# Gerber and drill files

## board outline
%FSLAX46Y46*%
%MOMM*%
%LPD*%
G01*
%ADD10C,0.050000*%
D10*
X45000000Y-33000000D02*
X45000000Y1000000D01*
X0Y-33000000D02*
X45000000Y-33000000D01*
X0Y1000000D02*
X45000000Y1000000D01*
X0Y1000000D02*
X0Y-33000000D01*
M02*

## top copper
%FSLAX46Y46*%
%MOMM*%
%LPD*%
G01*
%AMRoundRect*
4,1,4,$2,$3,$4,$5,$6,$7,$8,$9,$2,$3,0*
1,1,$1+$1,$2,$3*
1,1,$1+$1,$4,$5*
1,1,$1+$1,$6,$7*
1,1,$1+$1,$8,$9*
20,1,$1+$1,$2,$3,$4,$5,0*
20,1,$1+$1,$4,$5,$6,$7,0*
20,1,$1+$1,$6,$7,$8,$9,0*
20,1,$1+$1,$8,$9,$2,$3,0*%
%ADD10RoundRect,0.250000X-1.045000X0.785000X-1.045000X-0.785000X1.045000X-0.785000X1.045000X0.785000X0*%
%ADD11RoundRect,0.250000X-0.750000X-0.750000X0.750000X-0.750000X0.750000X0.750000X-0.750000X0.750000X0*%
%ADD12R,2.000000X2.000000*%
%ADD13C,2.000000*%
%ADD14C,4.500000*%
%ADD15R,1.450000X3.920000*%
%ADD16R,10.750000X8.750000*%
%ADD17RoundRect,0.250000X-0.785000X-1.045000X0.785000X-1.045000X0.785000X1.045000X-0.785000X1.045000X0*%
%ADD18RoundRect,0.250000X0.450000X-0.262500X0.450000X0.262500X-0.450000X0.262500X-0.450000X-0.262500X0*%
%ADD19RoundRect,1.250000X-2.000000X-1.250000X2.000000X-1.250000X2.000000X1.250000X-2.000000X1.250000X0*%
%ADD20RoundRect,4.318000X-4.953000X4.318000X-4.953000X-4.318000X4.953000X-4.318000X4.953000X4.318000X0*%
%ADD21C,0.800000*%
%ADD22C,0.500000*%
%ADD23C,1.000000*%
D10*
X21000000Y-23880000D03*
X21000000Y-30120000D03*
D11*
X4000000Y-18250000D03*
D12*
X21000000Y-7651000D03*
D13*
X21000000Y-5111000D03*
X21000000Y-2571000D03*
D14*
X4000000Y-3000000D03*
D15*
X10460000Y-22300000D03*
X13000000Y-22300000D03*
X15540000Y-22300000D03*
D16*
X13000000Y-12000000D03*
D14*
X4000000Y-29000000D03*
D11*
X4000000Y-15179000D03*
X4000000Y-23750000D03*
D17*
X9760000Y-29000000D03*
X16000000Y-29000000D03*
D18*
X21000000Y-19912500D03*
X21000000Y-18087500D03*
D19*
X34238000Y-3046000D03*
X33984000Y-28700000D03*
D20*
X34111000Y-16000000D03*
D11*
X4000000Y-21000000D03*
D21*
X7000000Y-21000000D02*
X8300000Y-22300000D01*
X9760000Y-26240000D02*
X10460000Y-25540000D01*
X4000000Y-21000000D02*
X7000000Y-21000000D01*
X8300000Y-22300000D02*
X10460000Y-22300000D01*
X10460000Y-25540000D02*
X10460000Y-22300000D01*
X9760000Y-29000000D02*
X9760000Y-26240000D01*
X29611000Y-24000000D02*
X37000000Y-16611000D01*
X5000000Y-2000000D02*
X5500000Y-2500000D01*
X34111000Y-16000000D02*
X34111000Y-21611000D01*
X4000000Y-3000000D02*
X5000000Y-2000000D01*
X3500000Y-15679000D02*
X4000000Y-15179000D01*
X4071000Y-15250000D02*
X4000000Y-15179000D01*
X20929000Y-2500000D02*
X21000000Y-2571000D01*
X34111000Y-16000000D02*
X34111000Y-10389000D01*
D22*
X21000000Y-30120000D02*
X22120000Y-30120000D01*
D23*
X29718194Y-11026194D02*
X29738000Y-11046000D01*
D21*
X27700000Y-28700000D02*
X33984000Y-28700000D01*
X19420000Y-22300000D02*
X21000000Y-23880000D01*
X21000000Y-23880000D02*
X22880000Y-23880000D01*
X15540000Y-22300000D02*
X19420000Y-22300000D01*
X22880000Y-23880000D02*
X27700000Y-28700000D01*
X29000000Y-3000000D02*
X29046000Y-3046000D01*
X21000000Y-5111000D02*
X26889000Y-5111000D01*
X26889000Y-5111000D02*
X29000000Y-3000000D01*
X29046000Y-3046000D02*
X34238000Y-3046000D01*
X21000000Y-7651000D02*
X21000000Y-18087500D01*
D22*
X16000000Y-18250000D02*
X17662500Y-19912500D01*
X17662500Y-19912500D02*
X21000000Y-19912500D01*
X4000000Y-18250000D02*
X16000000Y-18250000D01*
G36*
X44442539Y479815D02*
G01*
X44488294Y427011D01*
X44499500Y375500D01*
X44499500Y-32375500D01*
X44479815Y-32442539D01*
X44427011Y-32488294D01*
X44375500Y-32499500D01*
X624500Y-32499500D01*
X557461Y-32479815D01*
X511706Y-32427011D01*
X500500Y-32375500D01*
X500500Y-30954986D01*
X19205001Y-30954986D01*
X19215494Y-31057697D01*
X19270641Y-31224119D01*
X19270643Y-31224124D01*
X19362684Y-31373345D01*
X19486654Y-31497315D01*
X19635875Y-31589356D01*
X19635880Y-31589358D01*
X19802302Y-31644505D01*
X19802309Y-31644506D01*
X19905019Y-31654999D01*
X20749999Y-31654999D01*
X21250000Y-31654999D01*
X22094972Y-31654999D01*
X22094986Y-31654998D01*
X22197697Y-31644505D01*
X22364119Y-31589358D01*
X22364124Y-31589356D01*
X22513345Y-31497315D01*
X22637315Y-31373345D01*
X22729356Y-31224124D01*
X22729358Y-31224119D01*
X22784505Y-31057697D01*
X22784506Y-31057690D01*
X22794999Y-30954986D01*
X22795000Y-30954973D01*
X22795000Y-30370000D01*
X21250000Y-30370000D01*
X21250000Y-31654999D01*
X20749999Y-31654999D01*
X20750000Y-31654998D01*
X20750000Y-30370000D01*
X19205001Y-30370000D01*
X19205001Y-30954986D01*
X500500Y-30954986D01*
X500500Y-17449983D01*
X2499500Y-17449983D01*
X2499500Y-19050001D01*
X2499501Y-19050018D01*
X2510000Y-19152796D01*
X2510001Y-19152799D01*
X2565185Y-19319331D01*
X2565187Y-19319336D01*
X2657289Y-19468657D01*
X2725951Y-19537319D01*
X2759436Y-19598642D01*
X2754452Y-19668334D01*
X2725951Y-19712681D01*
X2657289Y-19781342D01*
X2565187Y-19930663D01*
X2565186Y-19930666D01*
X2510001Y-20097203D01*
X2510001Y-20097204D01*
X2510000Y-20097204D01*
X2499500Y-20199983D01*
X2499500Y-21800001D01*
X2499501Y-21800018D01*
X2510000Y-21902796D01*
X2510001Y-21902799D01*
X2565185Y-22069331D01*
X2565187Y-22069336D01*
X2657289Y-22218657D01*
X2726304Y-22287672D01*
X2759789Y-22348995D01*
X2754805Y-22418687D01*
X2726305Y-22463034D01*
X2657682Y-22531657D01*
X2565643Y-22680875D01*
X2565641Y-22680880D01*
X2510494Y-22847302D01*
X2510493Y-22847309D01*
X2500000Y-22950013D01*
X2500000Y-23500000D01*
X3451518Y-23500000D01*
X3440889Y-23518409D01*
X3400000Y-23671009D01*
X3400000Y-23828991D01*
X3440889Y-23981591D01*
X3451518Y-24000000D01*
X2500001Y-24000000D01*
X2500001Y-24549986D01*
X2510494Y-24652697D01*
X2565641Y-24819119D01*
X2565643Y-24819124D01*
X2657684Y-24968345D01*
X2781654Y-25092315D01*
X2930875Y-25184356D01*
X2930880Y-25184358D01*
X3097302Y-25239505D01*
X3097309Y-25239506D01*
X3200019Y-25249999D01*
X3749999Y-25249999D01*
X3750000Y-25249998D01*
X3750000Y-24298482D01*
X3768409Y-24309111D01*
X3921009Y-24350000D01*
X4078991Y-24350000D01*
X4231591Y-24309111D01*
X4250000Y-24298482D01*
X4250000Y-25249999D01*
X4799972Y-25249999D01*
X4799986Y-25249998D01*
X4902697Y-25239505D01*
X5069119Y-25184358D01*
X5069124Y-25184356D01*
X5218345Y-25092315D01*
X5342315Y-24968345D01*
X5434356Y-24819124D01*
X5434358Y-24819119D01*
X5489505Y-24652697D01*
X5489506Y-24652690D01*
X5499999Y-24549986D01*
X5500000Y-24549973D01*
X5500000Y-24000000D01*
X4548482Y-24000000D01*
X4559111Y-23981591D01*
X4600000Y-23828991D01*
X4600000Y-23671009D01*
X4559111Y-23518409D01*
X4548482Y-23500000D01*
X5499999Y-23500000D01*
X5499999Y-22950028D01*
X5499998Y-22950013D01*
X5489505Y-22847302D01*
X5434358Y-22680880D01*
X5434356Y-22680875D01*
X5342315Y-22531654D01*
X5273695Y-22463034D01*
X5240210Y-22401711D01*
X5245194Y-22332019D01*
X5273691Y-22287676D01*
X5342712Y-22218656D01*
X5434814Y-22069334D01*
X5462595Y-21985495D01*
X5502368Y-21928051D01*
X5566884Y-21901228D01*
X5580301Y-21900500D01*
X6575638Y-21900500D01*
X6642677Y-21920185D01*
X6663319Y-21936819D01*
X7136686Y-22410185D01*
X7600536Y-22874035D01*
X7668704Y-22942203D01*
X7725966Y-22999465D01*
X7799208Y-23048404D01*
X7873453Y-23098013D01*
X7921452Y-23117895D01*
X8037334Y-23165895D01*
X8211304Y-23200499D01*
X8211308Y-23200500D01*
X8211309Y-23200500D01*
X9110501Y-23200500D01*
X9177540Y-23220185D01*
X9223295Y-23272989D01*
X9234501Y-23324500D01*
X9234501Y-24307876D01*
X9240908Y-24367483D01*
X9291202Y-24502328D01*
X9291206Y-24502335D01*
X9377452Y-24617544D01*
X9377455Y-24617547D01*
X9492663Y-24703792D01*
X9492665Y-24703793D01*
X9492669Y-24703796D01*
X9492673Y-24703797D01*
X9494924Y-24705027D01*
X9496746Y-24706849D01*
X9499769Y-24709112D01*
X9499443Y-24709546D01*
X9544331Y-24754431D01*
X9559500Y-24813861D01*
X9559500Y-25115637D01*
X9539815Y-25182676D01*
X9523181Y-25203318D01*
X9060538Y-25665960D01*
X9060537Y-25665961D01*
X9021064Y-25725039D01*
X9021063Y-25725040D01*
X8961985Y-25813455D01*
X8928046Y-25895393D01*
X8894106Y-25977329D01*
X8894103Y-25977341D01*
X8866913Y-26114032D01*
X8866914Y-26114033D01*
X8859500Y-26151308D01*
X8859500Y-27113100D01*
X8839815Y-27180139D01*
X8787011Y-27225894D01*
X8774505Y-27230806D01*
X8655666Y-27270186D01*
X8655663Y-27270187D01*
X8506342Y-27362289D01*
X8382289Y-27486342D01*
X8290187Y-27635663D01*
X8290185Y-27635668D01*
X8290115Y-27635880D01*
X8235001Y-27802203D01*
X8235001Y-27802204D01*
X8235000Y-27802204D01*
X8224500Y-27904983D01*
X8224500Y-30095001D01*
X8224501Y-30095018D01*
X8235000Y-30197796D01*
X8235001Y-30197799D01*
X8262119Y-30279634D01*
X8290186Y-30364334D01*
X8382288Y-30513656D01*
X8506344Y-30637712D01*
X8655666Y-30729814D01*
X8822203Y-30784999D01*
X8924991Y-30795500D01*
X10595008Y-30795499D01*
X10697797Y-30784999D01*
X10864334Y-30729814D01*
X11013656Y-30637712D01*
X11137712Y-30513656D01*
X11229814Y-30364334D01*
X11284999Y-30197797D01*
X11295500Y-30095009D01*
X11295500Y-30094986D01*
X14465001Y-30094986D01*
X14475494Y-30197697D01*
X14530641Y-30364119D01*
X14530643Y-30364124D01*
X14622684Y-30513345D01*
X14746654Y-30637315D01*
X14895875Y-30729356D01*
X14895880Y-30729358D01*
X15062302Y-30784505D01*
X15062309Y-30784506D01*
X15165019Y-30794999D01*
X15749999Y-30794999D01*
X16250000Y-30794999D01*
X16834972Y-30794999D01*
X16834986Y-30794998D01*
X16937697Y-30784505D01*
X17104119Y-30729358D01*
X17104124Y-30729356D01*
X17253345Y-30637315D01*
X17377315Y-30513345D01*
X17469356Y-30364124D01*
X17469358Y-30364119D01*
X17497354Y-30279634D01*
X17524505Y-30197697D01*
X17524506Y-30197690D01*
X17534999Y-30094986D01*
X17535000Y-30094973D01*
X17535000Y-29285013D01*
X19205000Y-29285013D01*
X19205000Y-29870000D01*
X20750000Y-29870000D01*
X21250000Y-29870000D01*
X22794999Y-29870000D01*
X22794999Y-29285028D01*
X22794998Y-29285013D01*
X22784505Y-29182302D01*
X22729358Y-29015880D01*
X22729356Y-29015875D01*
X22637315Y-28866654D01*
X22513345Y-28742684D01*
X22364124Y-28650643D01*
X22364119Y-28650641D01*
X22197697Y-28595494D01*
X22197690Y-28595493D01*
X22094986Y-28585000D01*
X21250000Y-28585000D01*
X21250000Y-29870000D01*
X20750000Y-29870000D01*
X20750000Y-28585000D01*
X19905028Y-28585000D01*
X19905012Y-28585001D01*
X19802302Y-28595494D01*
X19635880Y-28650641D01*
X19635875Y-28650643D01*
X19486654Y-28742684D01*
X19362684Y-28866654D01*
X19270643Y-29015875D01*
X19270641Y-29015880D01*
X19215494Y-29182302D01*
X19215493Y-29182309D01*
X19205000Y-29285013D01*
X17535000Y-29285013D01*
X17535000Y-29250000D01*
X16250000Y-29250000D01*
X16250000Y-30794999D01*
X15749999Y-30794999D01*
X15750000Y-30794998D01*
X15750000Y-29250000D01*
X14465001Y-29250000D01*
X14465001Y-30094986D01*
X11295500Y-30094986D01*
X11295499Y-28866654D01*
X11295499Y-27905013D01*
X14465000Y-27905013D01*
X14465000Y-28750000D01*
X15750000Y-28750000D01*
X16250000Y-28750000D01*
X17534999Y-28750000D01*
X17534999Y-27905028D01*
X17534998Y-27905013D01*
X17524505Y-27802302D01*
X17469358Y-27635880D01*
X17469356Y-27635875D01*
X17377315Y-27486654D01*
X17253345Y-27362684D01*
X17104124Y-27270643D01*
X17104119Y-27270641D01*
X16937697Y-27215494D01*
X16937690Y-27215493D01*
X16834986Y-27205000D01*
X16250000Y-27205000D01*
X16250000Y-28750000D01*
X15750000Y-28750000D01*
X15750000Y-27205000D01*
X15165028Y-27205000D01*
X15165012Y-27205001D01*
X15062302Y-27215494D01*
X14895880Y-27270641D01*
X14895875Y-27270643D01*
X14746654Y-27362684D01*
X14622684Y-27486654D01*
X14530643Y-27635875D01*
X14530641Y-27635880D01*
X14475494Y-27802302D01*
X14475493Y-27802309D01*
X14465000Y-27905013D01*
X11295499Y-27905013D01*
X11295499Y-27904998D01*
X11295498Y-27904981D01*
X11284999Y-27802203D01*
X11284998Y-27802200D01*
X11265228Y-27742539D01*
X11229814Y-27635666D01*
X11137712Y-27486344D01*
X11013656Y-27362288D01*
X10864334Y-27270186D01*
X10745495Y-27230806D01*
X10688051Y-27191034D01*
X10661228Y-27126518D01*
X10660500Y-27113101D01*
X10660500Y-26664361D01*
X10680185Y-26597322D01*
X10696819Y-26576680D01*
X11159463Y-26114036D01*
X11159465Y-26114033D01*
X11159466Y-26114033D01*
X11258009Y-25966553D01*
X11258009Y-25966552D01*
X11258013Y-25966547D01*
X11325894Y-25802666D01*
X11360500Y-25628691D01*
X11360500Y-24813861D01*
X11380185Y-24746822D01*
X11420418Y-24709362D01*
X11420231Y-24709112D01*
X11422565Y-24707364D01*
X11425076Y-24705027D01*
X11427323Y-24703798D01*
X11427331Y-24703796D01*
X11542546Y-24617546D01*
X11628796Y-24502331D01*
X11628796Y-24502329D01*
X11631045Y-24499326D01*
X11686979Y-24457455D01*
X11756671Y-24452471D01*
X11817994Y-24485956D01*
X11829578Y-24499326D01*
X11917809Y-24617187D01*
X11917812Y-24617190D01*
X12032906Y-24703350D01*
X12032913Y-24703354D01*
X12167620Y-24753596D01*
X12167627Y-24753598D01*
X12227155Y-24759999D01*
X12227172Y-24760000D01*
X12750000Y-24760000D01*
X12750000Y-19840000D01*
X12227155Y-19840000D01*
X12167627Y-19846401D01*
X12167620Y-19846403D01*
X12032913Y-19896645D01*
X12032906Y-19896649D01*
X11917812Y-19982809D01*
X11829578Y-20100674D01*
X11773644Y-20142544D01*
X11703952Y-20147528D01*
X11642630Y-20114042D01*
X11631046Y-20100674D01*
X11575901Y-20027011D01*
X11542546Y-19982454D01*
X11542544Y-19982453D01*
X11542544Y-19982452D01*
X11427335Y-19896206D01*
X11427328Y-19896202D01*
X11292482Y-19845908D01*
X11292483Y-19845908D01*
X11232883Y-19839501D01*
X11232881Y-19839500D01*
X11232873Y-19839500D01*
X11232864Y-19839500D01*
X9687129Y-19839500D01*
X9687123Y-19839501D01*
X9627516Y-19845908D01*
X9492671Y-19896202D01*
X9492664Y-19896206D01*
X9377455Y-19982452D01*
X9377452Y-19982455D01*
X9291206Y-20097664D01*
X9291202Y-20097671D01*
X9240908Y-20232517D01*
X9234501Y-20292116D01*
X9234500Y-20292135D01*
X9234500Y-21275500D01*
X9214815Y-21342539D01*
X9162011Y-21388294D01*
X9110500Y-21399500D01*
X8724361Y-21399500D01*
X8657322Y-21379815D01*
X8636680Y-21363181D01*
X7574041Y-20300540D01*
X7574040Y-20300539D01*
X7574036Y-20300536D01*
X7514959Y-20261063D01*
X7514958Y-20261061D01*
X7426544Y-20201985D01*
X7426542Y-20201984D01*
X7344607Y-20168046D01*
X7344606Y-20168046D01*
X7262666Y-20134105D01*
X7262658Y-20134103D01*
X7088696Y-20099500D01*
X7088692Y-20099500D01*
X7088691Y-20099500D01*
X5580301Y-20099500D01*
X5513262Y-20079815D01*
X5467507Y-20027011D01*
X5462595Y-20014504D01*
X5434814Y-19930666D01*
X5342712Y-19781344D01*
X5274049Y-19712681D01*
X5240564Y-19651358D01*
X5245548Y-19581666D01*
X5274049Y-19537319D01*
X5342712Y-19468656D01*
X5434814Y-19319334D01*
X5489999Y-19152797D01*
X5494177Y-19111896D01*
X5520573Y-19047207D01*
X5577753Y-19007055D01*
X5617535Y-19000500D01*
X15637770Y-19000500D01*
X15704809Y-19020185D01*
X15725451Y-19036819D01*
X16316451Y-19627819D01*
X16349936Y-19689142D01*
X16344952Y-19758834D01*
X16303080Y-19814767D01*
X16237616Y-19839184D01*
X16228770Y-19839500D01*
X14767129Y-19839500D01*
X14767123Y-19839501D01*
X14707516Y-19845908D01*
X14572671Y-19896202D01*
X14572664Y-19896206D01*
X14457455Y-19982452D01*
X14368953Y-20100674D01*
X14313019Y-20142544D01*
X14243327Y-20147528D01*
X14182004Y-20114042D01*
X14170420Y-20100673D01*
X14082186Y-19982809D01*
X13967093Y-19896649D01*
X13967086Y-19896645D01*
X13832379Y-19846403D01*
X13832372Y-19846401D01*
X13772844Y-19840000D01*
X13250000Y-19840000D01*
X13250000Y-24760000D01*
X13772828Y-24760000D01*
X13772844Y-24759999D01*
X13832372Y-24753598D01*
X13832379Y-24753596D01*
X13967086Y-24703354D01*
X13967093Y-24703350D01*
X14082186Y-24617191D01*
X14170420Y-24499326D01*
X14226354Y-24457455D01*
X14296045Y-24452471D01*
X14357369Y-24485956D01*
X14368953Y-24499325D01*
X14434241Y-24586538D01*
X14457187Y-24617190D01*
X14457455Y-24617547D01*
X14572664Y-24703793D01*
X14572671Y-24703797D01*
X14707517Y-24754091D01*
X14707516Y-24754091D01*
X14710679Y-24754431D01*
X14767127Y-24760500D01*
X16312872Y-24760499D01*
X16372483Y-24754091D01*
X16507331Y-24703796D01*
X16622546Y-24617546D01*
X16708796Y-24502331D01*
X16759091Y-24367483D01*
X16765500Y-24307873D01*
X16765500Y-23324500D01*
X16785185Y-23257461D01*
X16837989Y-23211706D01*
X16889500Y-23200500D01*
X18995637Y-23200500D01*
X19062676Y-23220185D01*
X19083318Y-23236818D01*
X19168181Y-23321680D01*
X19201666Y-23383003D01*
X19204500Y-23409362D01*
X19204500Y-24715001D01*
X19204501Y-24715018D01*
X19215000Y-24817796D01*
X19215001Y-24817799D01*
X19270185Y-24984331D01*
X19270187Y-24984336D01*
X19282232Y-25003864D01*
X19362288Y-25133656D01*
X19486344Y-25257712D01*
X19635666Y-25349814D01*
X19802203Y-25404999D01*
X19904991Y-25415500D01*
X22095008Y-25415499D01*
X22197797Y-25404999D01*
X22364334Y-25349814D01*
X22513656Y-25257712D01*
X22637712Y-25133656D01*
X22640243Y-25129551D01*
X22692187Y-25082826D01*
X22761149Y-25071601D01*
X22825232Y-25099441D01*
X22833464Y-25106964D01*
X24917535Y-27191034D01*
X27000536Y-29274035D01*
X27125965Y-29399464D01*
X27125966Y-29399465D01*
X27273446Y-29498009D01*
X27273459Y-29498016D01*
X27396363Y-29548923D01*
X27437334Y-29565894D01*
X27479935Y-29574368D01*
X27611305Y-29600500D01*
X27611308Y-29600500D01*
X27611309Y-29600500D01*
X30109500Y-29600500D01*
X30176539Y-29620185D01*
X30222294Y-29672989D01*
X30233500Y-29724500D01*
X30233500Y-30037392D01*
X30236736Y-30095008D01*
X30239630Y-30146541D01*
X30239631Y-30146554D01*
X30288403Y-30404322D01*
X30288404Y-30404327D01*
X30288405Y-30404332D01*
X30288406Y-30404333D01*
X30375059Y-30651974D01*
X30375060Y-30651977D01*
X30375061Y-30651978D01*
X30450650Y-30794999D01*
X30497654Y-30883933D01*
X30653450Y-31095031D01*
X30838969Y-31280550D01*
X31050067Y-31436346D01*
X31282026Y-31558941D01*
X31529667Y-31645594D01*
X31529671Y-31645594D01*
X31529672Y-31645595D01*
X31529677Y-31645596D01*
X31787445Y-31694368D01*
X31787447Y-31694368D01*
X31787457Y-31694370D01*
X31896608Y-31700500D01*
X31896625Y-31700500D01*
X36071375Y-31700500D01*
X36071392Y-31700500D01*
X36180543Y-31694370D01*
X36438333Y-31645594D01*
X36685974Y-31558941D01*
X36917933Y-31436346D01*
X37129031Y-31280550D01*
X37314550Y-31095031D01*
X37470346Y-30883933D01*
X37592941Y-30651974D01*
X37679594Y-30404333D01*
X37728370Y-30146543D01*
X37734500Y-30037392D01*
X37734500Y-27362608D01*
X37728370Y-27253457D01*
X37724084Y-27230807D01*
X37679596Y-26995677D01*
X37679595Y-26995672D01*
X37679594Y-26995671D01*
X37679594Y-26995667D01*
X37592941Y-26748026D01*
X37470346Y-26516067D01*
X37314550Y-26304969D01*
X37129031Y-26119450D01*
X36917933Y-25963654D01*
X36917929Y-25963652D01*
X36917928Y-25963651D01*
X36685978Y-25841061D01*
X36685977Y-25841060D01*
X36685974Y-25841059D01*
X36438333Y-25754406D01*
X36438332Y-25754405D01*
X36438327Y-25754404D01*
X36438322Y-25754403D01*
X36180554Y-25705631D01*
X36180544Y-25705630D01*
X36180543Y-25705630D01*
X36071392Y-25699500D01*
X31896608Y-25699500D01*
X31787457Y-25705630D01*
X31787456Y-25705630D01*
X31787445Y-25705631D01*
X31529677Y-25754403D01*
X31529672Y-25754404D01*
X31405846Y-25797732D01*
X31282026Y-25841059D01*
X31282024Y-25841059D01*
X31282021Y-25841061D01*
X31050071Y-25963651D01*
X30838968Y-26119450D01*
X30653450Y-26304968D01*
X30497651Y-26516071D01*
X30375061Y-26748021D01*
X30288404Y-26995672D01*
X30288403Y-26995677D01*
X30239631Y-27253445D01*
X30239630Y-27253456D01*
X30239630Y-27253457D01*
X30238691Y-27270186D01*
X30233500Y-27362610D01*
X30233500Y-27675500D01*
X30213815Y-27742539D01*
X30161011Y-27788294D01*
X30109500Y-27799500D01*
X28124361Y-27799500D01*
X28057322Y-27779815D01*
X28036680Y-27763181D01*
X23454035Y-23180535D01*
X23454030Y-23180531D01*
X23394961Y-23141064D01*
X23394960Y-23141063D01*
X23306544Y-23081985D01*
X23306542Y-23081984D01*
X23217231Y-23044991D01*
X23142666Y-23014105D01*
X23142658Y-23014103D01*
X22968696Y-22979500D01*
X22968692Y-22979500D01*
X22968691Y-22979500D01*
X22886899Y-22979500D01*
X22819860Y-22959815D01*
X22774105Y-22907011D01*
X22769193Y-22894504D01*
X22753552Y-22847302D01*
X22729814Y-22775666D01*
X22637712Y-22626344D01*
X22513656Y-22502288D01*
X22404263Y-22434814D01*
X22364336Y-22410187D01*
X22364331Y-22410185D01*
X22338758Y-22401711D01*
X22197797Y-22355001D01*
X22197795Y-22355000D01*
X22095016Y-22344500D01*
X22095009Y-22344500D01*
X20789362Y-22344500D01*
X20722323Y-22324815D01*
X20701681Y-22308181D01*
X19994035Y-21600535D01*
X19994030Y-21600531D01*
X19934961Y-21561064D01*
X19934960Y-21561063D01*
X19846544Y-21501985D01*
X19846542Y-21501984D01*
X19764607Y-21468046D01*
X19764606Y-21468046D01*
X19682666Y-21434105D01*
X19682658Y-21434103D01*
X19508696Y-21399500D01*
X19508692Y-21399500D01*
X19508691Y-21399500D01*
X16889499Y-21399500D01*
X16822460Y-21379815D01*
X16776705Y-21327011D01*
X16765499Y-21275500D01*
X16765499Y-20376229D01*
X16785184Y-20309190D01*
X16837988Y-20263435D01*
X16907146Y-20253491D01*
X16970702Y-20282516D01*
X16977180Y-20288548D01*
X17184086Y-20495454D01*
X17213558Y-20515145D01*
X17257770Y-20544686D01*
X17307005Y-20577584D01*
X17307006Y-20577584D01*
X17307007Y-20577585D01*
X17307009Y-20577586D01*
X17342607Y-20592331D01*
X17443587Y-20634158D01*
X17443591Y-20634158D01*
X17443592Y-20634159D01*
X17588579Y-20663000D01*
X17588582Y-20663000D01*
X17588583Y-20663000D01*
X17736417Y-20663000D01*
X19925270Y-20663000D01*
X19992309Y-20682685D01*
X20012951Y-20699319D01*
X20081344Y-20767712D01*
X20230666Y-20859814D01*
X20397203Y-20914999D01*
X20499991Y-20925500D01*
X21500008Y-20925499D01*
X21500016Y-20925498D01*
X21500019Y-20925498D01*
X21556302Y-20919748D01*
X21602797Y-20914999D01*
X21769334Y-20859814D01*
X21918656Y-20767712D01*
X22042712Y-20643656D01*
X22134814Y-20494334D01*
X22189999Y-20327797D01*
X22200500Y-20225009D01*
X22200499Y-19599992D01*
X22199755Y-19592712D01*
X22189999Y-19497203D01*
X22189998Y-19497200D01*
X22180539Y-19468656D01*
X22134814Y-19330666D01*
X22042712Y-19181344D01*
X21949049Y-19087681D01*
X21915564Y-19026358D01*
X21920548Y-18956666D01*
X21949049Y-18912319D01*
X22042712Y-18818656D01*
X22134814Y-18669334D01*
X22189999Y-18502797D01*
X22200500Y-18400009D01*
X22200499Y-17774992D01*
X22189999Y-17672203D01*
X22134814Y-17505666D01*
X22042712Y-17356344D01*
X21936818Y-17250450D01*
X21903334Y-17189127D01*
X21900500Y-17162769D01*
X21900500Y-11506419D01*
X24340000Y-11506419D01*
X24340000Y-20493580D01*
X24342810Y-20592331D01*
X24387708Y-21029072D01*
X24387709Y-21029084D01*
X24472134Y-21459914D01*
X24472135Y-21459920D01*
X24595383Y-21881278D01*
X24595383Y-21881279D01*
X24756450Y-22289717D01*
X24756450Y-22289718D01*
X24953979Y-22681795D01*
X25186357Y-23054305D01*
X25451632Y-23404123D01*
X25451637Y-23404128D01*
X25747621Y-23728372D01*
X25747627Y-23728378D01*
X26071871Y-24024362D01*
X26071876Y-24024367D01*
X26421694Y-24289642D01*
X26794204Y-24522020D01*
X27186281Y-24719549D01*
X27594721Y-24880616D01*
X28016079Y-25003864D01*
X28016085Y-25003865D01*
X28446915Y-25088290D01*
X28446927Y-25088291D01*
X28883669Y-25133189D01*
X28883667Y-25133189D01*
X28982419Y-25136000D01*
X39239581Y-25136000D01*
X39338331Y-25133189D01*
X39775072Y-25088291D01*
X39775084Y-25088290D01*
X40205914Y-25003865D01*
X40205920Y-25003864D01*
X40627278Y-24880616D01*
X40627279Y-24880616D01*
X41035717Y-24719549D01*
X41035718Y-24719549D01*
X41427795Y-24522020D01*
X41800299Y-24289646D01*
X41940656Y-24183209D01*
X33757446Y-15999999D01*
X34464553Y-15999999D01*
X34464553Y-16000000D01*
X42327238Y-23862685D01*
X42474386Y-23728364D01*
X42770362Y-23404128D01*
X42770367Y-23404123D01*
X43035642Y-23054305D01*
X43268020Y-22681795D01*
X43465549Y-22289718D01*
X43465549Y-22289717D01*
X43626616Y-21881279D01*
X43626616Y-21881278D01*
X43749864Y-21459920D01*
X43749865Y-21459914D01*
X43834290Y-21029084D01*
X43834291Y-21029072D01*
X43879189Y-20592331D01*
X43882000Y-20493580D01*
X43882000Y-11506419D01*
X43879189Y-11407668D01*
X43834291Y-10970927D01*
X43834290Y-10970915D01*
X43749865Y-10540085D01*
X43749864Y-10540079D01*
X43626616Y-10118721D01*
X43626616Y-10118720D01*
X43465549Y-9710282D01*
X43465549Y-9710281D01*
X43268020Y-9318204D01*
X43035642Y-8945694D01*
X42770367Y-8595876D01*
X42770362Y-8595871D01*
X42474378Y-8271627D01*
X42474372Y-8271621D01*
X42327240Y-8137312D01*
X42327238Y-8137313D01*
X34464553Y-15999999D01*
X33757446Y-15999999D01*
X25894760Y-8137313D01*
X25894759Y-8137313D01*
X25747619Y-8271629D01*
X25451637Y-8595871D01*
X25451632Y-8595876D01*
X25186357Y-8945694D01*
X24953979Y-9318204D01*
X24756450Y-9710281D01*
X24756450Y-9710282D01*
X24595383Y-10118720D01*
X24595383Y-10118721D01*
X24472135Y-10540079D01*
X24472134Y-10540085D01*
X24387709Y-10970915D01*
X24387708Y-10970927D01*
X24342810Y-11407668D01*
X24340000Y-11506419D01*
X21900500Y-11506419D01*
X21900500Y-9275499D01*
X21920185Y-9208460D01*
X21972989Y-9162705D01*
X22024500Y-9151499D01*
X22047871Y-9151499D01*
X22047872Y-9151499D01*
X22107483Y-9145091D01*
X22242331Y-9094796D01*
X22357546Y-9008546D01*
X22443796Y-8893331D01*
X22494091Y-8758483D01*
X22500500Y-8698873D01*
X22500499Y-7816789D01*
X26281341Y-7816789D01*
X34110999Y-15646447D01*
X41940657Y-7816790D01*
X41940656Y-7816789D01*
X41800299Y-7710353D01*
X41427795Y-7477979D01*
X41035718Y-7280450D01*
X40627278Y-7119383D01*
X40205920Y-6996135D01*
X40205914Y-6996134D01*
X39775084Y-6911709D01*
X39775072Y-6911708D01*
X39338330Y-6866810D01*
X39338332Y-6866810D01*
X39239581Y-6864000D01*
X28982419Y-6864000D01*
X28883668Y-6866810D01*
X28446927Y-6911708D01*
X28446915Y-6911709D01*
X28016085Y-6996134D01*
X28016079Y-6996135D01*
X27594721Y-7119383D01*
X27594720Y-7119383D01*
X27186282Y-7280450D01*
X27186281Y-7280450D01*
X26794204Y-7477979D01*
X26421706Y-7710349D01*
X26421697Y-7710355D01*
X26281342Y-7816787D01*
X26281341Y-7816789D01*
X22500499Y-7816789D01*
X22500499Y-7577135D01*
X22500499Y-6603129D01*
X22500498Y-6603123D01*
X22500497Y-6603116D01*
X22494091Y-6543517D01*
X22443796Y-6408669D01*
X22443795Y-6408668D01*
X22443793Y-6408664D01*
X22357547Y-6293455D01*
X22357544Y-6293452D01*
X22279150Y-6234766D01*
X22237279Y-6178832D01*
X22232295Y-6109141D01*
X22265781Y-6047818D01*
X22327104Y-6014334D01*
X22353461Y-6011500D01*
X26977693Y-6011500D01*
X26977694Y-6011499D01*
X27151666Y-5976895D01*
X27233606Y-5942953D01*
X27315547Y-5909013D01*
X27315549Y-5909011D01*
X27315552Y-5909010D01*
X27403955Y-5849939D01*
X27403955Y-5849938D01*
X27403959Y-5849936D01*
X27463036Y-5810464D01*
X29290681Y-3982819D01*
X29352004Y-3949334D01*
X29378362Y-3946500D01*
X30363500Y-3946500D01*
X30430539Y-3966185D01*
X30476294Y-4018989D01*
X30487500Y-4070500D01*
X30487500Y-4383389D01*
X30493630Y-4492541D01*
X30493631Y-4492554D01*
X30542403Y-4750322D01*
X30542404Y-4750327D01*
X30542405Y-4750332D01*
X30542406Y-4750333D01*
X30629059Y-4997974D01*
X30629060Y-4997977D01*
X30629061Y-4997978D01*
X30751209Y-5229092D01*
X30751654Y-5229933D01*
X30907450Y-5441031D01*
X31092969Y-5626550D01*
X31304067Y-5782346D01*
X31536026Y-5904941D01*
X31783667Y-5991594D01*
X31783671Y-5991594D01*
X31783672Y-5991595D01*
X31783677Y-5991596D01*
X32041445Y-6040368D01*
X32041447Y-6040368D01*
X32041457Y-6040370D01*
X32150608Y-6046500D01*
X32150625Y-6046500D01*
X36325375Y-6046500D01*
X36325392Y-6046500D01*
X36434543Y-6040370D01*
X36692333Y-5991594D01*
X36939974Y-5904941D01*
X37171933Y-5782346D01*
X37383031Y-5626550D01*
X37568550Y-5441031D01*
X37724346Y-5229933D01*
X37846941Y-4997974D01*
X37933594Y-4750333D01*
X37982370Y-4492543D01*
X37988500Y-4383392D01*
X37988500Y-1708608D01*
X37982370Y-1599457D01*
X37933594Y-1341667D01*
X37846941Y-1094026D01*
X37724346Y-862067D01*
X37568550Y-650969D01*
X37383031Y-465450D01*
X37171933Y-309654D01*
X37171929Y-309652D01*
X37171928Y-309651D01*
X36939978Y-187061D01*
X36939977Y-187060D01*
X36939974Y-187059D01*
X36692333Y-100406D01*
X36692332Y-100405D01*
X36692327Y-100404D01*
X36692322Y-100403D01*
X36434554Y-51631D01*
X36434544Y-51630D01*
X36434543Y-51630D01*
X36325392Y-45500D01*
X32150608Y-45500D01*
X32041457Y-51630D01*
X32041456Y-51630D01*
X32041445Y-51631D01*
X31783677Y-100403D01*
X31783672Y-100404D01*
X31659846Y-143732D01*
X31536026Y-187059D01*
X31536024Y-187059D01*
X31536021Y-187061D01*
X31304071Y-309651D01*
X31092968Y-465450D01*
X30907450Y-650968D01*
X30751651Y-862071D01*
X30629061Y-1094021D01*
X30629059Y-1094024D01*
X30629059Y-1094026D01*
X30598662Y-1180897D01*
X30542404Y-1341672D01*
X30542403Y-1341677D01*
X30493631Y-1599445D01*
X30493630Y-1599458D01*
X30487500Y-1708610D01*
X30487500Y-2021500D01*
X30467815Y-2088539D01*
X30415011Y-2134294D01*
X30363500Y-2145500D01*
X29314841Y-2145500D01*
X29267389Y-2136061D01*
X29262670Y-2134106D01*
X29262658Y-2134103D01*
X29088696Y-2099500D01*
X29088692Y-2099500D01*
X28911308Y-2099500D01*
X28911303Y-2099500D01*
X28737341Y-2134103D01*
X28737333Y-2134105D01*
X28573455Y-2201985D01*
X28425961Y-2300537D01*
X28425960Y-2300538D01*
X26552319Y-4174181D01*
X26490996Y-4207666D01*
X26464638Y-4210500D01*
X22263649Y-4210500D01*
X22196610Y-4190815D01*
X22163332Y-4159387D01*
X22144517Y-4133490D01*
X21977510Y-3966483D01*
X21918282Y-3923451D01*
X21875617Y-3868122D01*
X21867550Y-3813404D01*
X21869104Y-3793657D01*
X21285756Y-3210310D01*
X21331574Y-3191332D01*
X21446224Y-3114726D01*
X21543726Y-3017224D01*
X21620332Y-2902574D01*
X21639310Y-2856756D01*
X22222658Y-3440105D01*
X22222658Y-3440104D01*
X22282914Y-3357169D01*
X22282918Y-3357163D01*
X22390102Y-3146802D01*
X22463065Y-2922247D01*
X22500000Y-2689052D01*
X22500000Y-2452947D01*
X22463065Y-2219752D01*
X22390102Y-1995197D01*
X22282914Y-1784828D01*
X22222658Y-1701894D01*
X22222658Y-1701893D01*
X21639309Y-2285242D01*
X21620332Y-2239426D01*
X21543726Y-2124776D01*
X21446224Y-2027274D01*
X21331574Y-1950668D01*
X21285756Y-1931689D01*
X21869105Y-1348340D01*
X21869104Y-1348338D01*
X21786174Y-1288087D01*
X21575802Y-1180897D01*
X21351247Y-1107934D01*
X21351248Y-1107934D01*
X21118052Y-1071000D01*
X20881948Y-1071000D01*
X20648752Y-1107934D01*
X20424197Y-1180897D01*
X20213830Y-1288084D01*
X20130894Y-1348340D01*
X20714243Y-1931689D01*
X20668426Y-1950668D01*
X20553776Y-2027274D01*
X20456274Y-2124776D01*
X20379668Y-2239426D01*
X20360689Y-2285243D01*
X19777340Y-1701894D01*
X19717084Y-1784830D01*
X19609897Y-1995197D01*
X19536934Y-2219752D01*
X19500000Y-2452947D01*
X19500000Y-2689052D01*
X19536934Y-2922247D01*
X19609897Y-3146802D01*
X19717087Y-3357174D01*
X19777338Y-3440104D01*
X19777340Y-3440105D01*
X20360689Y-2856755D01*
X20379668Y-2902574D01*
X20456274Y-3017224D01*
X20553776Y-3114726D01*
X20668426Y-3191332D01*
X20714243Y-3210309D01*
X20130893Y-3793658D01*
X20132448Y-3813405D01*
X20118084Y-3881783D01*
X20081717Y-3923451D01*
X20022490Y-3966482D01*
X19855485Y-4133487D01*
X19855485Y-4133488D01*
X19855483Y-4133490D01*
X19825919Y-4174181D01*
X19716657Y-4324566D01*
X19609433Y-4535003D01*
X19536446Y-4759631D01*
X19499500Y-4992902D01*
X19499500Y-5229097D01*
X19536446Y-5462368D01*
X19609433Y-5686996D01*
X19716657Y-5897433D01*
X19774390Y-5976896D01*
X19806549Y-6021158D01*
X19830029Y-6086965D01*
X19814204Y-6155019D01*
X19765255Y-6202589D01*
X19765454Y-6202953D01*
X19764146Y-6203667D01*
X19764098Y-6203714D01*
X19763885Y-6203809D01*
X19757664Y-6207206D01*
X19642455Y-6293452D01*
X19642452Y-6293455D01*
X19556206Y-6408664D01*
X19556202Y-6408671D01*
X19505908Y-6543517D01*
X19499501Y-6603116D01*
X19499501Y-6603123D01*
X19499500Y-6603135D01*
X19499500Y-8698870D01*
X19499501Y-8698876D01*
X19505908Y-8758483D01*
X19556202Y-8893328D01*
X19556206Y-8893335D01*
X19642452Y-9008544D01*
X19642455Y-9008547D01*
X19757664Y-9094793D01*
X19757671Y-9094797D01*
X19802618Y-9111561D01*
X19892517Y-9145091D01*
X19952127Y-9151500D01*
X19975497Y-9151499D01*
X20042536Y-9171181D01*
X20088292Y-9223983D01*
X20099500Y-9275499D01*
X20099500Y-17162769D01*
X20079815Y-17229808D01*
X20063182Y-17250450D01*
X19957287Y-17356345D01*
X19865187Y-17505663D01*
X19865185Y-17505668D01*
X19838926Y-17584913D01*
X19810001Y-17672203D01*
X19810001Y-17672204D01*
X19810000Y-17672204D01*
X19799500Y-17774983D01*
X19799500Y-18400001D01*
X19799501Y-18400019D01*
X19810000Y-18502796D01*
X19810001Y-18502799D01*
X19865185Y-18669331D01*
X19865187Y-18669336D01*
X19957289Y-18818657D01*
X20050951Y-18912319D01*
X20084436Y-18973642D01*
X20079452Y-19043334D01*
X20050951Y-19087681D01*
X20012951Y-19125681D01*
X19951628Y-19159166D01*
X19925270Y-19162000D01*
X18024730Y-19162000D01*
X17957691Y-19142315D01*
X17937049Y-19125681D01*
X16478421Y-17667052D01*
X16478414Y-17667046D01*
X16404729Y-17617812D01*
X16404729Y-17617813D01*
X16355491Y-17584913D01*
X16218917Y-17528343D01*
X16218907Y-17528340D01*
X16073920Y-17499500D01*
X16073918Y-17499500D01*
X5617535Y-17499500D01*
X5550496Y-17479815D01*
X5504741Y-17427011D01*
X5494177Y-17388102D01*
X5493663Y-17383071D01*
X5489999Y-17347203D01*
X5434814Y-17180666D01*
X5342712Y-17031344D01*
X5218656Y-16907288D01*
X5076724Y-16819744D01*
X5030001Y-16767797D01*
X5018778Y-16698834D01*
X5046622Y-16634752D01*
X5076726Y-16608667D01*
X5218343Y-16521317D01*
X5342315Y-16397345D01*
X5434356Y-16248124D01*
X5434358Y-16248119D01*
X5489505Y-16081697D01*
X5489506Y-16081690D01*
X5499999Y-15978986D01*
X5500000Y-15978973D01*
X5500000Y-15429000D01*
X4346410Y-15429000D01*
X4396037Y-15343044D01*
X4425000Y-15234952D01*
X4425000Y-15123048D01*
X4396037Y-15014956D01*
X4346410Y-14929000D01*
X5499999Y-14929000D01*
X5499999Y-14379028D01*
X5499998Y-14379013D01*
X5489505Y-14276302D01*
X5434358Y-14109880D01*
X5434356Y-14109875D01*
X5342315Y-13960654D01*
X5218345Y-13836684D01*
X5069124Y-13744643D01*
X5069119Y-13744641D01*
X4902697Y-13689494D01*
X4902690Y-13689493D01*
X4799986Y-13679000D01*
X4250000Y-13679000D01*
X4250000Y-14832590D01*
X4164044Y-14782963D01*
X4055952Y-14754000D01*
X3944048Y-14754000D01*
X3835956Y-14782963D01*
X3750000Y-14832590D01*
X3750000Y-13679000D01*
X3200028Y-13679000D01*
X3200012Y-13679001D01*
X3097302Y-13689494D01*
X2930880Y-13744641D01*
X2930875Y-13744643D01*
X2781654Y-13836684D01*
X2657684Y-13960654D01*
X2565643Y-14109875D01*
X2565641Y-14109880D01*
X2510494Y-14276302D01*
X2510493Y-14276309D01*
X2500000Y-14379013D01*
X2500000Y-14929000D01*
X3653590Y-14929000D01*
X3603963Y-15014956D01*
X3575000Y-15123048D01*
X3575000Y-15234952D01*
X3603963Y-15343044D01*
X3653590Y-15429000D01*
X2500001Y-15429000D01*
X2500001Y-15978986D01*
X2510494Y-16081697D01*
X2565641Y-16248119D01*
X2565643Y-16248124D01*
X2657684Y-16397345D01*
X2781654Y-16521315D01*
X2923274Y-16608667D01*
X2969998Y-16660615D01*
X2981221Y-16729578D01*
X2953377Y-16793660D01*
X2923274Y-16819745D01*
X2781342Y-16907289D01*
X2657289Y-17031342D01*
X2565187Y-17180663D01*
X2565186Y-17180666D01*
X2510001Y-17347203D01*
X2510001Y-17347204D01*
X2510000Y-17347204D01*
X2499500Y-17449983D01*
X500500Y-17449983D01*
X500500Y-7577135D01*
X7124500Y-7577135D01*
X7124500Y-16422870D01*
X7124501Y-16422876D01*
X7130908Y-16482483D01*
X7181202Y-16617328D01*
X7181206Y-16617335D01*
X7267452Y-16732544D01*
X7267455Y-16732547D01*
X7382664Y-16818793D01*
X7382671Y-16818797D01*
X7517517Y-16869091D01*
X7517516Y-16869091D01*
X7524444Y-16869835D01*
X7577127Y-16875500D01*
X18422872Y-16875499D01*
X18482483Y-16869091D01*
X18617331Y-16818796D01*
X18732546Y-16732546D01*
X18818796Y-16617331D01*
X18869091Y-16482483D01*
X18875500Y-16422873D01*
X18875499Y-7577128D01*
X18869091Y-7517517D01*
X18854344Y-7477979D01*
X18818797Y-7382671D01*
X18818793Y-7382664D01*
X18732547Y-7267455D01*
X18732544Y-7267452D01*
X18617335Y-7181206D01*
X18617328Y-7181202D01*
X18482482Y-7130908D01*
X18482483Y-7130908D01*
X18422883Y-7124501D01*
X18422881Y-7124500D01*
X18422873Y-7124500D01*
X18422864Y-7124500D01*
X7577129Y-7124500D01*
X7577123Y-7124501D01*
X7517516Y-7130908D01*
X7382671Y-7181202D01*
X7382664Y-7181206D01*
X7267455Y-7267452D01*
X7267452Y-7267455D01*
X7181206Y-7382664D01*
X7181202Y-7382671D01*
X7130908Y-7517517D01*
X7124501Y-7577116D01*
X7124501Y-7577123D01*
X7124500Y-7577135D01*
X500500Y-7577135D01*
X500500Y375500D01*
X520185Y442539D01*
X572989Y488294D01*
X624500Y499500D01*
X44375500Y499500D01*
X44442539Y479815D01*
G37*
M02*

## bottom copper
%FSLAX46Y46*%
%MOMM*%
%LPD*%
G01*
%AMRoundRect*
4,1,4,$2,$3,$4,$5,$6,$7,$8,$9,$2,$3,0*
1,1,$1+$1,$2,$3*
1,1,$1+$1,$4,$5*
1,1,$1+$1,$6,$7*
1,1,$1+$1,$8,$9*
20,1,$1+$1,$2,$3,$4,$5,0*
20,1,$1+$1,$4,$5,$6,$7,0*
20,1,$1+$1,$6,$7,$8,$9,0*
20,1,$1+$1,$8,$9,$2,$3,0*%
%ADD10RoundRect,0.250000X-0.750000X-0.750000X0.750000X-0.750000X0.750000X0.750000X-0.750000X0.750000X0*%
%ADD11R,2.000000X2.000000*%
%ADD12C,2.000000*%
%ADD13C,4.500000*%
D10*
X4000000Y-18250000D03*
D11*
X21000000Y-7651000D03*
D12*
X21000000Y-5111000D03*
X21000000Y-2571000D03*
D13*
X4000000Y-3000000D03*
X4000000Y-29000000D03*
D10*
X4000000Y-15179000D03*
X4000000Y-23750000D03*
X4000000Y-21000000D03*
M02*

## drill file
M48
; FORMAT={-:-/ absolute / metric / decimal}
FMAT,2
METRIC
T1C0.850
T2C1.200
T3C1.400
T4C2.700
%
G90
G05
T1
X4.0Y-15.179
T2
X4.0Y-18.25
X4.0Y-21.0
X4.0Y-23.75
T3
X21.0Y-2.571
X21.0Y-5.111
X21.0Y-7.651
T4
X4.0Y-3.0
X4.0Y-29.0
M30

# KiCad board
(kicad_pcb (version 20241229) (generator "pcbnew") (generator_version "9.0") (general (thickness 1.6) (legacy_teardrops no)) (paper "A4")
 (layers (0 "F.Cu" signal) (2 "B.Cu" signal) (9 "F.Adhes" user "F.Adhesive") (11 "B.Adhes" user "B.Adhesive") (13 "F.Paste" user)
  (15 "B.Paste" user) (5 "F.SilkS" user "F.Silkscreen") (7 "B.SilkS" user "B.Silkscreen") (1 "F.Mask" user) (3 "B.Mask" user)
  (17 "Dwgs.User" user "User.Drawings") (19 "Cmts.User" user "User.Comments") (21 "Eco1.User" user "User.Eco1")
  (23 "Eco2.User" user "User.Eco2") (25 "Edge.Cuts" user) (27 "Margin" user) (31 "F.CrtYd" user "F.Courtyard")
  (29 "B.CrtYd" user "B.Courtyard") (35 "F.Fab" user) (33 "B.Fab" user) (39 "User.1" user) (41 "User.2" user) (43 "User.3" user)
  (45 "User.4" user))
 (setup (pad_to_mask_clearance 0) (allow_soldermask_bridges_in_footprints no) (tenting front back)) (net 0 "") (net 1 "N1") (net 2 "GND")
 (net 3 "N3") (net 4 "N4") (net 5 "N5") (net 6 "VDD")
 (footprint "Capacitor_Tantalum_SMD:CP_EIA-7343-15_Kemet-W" (layer "F.Cu") (at 21 27 -90)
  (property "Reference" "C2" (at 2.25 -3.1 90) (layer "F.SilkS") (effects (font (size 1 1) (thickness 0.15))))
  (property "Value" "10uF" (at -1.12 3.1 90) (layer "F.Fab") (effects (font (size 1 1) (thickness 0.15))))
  (pad "1" smd roundrect (at -3.12 0 270) (size 2.07 2.59) (layers "F.Cu" "F.Mask" "F.Paste") (roundrect_rratio 0.120773) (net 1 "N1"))
  (pad "2" smd roundrect (at 3.12 0 270) (size 2.07 2.59) (layers "F.Cu" "F.Mask" "F.Paste") (roundrect_rratio 0.120773) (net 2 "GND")))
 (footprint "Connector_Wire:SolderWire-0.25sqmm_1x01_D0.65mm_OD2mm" (layer "F.Cu") (at 4 18.25)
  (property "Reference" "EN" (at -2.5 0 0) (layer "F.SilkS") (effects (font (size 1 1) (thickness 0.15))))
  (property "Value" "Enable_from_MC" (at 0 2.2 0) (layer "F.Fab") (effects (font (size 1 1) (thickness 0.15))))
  (pad "1" thru_hole roundrect (at 0 0) (size 2 2) (drill 1.2) (layers "*.Cu" "*.Mask") (remove_unused_layers no) (roundrect_rratio 0.125)
   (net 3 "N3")))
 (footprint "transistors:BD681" (layer "F.Cu") (at 21 7.651 90)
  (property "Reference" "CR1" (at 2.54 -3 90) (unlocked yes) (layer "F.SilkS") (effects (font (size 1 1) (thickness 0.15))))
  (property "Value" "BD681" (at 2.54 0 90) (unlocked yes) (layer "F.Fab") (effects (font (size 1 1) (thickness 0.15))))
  (pad "1" thru_hole rect (at 0 0 90) (size 2 2) (drill 1.4) (layers "*.Cu" "*.Mask") (remove_unused_layers no) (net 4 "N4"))
  (pad "2" thru_hole circle (at 2.54 0 90) (size 2 2) (drill 1.4) (layers "*.Cu" "*.Mask") (remove_unused_layers no) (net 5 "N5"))
  (pad "3" thru_hole circle (at 5.08 0 90) (size 2 2) (drill 1.4) (layers "*.Cu" "*.Mask") (remove_unused_layers no) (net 2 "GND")))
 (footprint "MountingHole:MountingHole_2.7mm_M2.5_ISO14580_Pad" (layer "F.Cu") (at 4 3)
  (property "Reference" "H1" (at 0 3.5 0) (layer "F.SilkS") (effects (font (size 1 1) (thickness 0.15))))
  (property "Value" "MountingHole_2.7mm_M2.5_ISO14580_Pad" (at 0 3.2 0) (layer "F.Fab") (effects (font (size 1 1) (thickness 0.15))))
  (pad "1" thru_hole circle (at 0 0) (size 4.5 4.5) (drill 2.7) (layers "*.Cu" "*.Mask") (remove_unused_layers no) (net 2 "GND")
   (zone_connect 2)))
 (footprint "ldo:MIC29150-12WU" (layer "F.Cu") (at 13 15.95 90)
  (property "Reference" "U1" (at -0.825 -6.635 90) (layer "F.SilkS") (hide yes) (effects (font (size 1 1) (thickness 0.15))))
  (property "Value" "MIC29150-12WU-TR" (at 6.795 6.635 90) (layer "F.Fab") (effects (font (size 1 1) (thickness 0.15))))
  (pad "1" smd rect (at -6.35 -2.54 90) (size 3.92 1.45) (layers "F.Cu" "F.Mask" "F.Paste") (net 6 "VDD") (solder_mask_margin 0.102))
  (pad "2" smd rect (at -6.35 0 90) (size 3.92 1.45) (layers "F.Cu" "F.Mask" "F.Paste") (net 2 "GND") (solder_mask_margin 0.102))
  (pad "3" smd rect (at -6.35 2.54 90) (size 3.92 1.45) (layers "F.Cu" "F.Mask" "F.Paste") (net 1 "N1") (solder_mask_margin 0.102))
  (pad "4" smd rect (at 3.95 0 90) (size 8.75 10.75) (layers "F.Cu" "F.Mask") (solder_mask_margin 0.102)))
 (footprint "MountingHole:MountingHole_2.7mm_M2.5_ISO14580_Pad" (layer "F.Cu") (at 4 29)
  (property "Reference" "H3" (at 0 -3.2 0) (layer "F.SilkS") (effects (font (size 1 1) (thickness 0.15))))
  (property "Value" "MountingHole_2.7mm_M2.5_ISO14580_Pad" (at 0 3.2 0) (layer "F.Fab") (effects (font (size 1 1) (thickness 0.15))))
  (pad "3" thru_hole circle (at 0 0) (size 4.5 4.5) (drill 2.7) (layers "*.Cu" "*.Mask") (remove_unused_layers no) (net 2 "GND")
   (zone_connect 2)))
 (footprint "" (layer "F.Cu") (at 4 15.179)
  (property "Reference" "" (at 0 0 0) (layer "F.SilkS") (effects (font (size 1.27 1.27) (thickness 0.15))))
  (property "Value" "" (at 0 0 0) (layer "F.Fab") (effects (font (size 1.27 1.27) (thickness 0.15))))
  (pad "GND_PIN" thru_hole roundrect (at 0 0) (size 2 2) (drill 0.85) (layers "*.Cu" "*.Mask") (remove_unused_layers no)
   (roundrect_rratio 0.125) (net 2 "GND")))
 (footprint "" (layer "F.Cu") (at 4 23.75)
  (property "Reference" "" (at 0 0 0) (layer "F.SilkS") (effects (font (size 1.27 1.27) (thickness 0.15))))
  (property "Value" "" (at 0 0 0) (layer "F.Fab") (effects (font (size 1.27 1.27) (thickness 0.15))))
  (pad "GND_PIN" thru_hole roundrect (at 0 0) (size 2 2) (drill 1.2) (layers "*.Cu" "*.Mask") (remove_unused_layers no)
   (roundrect_rratio 0.125) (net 2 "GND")))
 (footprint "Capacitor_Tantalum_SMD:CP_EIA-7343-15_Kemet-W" (layer "F.Cu") (at 12.88 29)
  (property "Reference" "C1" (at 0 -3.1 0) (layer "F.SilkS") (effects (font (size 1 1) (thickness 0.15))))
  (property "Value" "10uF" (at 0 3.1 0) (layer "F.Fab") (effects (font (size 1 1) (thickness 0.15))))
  (pad "1" smd roundrect (at -3.12 0) (size 2.07 2.59) (layers "F.Cu" "F.Mask" "F.Paste") (roundrect_rratio 0.120773) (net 6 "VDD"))
  (pad "2" smd roundrect (at 3.12 0) (size 2.07 2.59) (layers "F.Cu" "F.Mask" "F.Paste") (roundrect_rratio 0.120773) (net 2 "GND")))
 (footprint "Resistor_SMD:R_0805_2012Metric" (layer "F.Cu") (at 21 19 90)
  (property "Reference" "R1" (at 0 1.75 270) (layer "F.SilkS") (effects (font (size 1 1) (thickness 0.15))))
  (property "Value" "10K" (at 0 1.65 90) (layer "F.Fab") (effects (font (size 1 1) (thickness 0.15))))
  (pad "1" smd roundrect (at -0.9125 0 90) (size 1.025 1.4) (layers "F.Cu" "F.Mask" "F.Paste") (roundrect_rratio 0.243902) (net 3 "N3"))
  (pad "2" smd roundrect (at 0.9125 0 90) (size 1.025 1.4) (layers "F.Cu" "F.Mask" "F.Paste") (roundrect_rratio 0.243902) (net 4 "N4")))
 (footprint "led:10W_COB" (layer "F.Cu") (at 35 16 -90)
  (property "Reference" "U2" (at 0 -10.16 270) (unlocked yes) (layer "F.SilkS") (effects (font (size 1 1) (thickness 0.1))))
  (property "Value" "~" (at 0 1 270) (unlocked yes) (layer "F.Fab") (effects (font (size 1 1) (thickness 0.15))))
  (pad "1" smd roundrect (at -12.954 0.762) (size 6.5 5) (layers "F.Cu" "F.Mask" "F.Paste") (roundrect_rratio 0.25) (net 5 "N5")
   (thermal_bridge_angle 45))
  (pad "2" smd roundrect (at 12.7 1.016) (size 6.5 5) (layers "F.Cu" "F.Mask" "F.Paste") (roundrect_rratio 0.25) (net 1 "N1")
   (thermal_bridge_angle 45))
  (pad "3" smd roundrect (at 0 0.889 270) (size 17.272 18.542) (layers "F.Cu" "F.Mask" "F.Paste") (roundrect_rratio 0.25) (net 2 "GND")
   (thermal_bridge_angle 45)))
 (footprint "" (layer "F.Cu") (at 4 21)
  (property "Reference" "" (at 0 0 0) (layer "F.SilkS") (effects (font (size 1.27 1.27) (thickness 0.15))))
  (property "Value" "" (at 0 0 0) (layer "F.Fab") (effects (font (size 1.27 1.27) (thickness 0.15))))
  (pad "VDD_PIN" thru_hole roundrect (at 0 0) (size 2 2) (drill 1.2) (layers "*.Cu" "*.Mask") (remove_unused_layers no)
   (roundrect_rratio 0.125) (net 6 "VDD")))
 (gr_line (start 45 33) (end 45 -1) (stroke (width 0.05) (type default)) (layer "Edge.Cuts"))
 (gr_line (start 0 33) (end 45 33) (stroke (width 0.05) (type default)) (layer "Edge.Cuts"))
 (gr_line (start 0 -1) (end 45 -1) (stroke (width 0.05) (type default)) (layer "Edge.Cuts"))
 (gr_line (start 0 -1) (end 0 33) (stroke (width 0.05) (type default)) (layer "Edge.Cuts"))
 (segment (start 7 21) (end 8.3 22.3) (width 0.8) (layer "F.Cu") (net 6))
 (segment (start 9.76 26.24) (end 10.46 25.54) (width 0.8) (layer "F.Cu") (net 6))
 (segment (start 4 21) (end 7 21) (width 0.8) (layer "F.Cu") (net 6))
 (segment (start 8.3 22.3) (end 10.46 22.3) (width 0.8) (layer "F.Cu") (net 6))
 (segment (start 10.46 25.54) (end 10.46 22.3) (width 0.8) (layer "F.Cu") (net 6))
 (segment (start 9.76 29) (end 9.76 26.24) (width 0.8) (layer "F.Cu") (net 6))
 (segment (start 29.611 24) (end 37 16.611) (width 0.8) (layer "F.Cu") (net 2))
 (segment (start 5 2) (end 5.5 2.5) (width 0.8) (layer "F.Cu") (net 2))
 (segment (start 34.111 16) (end 34.111 21.611) (width 0.8) (layer "F.Cu") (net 2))
 (segment (start 4 3) (end 5 2) (width 0.8) (layer "F.Cu") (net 2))
 (segment (start 3.5 15.679) (end 4 15.179) (width 0.8) (layer "F.Cu") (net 2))
 (segment (start 4.071 15.25) (end 4 15.179) (width 0.8) (layer "F.Cu") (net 2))
 (segment (start 20.929 2.5) (end 21 2.571) (width 0.8) (layer "F.Cu") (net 2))
 (segment (start 34.111 16) (end 34.111 10.389) (width 0.8) (layer "F.Cu") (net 2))
 (segment (start 21 30.12) (end 22.12 30.12) (width 0.5) (layer "F.Cu") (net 2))
 (segment (start 29.718194 11.026194) (end 29.738 11.046) (width 1) (layer "F.Cu") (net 2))
 (segment (start 27.7 28.7) (end 33.984 28.7) (width 0.8) (layer "F.Cu") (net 1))
 (segment (start 19.42 22.3) (end 21 23.88) (width 0.8) (layer "F.Cu") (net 1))
 (segment (start 21 23.88) (end 22.88 23.88) (width 0.8) (layer "F.Cu") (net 1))
 (segment (start 15.54 22.3) (end 19.42 22.3) (width 0.8) (layer "F.Cu") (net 1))
 (segment (start 22.88 23.88) (end 27.7 28.7) (width 0.8) (layer "F.Cu") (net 1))
 (segment (start 29 3) (end 29.046 3.046) (width 0.8) (layer "F.Cu") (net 5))
 (segment (start 21 5.111) (end 26.889 5.111) (width 0.8) (layer "F.Cu") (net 5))
 (segment (start 26.889 5.111) (end 29 3) (width 0.8) (layer "F.Cu") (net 5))
 (segment (start 29.046 3.046) (end 34.238 3.046) (width 0.8) (layer "F.Cu") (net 5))
 (segment (start 21 7.651) (end 21 18.0875) (width 0.8) (layer "F.Cu") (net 4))
 (segment (start 16 18.25) (end 17.6625 19.9125) (width 0.5) (layer "F.Cu") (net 3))
 (segment (start 17.6625 19.9125) (end 21 19.9125) (width 0.5) (layer "F.Cu") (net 3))
 (segment (start 4 18.25) (end 16 18.25) (width 0.5) (layer "F.Cu") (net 3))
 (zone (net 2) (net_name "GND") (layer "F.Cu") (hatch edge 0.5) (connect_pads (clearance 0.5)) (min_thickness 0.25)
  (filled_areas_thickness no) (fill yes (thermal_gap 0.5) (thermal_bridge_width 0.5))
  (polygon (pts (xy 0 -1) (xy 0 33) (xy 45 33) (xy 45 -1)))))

